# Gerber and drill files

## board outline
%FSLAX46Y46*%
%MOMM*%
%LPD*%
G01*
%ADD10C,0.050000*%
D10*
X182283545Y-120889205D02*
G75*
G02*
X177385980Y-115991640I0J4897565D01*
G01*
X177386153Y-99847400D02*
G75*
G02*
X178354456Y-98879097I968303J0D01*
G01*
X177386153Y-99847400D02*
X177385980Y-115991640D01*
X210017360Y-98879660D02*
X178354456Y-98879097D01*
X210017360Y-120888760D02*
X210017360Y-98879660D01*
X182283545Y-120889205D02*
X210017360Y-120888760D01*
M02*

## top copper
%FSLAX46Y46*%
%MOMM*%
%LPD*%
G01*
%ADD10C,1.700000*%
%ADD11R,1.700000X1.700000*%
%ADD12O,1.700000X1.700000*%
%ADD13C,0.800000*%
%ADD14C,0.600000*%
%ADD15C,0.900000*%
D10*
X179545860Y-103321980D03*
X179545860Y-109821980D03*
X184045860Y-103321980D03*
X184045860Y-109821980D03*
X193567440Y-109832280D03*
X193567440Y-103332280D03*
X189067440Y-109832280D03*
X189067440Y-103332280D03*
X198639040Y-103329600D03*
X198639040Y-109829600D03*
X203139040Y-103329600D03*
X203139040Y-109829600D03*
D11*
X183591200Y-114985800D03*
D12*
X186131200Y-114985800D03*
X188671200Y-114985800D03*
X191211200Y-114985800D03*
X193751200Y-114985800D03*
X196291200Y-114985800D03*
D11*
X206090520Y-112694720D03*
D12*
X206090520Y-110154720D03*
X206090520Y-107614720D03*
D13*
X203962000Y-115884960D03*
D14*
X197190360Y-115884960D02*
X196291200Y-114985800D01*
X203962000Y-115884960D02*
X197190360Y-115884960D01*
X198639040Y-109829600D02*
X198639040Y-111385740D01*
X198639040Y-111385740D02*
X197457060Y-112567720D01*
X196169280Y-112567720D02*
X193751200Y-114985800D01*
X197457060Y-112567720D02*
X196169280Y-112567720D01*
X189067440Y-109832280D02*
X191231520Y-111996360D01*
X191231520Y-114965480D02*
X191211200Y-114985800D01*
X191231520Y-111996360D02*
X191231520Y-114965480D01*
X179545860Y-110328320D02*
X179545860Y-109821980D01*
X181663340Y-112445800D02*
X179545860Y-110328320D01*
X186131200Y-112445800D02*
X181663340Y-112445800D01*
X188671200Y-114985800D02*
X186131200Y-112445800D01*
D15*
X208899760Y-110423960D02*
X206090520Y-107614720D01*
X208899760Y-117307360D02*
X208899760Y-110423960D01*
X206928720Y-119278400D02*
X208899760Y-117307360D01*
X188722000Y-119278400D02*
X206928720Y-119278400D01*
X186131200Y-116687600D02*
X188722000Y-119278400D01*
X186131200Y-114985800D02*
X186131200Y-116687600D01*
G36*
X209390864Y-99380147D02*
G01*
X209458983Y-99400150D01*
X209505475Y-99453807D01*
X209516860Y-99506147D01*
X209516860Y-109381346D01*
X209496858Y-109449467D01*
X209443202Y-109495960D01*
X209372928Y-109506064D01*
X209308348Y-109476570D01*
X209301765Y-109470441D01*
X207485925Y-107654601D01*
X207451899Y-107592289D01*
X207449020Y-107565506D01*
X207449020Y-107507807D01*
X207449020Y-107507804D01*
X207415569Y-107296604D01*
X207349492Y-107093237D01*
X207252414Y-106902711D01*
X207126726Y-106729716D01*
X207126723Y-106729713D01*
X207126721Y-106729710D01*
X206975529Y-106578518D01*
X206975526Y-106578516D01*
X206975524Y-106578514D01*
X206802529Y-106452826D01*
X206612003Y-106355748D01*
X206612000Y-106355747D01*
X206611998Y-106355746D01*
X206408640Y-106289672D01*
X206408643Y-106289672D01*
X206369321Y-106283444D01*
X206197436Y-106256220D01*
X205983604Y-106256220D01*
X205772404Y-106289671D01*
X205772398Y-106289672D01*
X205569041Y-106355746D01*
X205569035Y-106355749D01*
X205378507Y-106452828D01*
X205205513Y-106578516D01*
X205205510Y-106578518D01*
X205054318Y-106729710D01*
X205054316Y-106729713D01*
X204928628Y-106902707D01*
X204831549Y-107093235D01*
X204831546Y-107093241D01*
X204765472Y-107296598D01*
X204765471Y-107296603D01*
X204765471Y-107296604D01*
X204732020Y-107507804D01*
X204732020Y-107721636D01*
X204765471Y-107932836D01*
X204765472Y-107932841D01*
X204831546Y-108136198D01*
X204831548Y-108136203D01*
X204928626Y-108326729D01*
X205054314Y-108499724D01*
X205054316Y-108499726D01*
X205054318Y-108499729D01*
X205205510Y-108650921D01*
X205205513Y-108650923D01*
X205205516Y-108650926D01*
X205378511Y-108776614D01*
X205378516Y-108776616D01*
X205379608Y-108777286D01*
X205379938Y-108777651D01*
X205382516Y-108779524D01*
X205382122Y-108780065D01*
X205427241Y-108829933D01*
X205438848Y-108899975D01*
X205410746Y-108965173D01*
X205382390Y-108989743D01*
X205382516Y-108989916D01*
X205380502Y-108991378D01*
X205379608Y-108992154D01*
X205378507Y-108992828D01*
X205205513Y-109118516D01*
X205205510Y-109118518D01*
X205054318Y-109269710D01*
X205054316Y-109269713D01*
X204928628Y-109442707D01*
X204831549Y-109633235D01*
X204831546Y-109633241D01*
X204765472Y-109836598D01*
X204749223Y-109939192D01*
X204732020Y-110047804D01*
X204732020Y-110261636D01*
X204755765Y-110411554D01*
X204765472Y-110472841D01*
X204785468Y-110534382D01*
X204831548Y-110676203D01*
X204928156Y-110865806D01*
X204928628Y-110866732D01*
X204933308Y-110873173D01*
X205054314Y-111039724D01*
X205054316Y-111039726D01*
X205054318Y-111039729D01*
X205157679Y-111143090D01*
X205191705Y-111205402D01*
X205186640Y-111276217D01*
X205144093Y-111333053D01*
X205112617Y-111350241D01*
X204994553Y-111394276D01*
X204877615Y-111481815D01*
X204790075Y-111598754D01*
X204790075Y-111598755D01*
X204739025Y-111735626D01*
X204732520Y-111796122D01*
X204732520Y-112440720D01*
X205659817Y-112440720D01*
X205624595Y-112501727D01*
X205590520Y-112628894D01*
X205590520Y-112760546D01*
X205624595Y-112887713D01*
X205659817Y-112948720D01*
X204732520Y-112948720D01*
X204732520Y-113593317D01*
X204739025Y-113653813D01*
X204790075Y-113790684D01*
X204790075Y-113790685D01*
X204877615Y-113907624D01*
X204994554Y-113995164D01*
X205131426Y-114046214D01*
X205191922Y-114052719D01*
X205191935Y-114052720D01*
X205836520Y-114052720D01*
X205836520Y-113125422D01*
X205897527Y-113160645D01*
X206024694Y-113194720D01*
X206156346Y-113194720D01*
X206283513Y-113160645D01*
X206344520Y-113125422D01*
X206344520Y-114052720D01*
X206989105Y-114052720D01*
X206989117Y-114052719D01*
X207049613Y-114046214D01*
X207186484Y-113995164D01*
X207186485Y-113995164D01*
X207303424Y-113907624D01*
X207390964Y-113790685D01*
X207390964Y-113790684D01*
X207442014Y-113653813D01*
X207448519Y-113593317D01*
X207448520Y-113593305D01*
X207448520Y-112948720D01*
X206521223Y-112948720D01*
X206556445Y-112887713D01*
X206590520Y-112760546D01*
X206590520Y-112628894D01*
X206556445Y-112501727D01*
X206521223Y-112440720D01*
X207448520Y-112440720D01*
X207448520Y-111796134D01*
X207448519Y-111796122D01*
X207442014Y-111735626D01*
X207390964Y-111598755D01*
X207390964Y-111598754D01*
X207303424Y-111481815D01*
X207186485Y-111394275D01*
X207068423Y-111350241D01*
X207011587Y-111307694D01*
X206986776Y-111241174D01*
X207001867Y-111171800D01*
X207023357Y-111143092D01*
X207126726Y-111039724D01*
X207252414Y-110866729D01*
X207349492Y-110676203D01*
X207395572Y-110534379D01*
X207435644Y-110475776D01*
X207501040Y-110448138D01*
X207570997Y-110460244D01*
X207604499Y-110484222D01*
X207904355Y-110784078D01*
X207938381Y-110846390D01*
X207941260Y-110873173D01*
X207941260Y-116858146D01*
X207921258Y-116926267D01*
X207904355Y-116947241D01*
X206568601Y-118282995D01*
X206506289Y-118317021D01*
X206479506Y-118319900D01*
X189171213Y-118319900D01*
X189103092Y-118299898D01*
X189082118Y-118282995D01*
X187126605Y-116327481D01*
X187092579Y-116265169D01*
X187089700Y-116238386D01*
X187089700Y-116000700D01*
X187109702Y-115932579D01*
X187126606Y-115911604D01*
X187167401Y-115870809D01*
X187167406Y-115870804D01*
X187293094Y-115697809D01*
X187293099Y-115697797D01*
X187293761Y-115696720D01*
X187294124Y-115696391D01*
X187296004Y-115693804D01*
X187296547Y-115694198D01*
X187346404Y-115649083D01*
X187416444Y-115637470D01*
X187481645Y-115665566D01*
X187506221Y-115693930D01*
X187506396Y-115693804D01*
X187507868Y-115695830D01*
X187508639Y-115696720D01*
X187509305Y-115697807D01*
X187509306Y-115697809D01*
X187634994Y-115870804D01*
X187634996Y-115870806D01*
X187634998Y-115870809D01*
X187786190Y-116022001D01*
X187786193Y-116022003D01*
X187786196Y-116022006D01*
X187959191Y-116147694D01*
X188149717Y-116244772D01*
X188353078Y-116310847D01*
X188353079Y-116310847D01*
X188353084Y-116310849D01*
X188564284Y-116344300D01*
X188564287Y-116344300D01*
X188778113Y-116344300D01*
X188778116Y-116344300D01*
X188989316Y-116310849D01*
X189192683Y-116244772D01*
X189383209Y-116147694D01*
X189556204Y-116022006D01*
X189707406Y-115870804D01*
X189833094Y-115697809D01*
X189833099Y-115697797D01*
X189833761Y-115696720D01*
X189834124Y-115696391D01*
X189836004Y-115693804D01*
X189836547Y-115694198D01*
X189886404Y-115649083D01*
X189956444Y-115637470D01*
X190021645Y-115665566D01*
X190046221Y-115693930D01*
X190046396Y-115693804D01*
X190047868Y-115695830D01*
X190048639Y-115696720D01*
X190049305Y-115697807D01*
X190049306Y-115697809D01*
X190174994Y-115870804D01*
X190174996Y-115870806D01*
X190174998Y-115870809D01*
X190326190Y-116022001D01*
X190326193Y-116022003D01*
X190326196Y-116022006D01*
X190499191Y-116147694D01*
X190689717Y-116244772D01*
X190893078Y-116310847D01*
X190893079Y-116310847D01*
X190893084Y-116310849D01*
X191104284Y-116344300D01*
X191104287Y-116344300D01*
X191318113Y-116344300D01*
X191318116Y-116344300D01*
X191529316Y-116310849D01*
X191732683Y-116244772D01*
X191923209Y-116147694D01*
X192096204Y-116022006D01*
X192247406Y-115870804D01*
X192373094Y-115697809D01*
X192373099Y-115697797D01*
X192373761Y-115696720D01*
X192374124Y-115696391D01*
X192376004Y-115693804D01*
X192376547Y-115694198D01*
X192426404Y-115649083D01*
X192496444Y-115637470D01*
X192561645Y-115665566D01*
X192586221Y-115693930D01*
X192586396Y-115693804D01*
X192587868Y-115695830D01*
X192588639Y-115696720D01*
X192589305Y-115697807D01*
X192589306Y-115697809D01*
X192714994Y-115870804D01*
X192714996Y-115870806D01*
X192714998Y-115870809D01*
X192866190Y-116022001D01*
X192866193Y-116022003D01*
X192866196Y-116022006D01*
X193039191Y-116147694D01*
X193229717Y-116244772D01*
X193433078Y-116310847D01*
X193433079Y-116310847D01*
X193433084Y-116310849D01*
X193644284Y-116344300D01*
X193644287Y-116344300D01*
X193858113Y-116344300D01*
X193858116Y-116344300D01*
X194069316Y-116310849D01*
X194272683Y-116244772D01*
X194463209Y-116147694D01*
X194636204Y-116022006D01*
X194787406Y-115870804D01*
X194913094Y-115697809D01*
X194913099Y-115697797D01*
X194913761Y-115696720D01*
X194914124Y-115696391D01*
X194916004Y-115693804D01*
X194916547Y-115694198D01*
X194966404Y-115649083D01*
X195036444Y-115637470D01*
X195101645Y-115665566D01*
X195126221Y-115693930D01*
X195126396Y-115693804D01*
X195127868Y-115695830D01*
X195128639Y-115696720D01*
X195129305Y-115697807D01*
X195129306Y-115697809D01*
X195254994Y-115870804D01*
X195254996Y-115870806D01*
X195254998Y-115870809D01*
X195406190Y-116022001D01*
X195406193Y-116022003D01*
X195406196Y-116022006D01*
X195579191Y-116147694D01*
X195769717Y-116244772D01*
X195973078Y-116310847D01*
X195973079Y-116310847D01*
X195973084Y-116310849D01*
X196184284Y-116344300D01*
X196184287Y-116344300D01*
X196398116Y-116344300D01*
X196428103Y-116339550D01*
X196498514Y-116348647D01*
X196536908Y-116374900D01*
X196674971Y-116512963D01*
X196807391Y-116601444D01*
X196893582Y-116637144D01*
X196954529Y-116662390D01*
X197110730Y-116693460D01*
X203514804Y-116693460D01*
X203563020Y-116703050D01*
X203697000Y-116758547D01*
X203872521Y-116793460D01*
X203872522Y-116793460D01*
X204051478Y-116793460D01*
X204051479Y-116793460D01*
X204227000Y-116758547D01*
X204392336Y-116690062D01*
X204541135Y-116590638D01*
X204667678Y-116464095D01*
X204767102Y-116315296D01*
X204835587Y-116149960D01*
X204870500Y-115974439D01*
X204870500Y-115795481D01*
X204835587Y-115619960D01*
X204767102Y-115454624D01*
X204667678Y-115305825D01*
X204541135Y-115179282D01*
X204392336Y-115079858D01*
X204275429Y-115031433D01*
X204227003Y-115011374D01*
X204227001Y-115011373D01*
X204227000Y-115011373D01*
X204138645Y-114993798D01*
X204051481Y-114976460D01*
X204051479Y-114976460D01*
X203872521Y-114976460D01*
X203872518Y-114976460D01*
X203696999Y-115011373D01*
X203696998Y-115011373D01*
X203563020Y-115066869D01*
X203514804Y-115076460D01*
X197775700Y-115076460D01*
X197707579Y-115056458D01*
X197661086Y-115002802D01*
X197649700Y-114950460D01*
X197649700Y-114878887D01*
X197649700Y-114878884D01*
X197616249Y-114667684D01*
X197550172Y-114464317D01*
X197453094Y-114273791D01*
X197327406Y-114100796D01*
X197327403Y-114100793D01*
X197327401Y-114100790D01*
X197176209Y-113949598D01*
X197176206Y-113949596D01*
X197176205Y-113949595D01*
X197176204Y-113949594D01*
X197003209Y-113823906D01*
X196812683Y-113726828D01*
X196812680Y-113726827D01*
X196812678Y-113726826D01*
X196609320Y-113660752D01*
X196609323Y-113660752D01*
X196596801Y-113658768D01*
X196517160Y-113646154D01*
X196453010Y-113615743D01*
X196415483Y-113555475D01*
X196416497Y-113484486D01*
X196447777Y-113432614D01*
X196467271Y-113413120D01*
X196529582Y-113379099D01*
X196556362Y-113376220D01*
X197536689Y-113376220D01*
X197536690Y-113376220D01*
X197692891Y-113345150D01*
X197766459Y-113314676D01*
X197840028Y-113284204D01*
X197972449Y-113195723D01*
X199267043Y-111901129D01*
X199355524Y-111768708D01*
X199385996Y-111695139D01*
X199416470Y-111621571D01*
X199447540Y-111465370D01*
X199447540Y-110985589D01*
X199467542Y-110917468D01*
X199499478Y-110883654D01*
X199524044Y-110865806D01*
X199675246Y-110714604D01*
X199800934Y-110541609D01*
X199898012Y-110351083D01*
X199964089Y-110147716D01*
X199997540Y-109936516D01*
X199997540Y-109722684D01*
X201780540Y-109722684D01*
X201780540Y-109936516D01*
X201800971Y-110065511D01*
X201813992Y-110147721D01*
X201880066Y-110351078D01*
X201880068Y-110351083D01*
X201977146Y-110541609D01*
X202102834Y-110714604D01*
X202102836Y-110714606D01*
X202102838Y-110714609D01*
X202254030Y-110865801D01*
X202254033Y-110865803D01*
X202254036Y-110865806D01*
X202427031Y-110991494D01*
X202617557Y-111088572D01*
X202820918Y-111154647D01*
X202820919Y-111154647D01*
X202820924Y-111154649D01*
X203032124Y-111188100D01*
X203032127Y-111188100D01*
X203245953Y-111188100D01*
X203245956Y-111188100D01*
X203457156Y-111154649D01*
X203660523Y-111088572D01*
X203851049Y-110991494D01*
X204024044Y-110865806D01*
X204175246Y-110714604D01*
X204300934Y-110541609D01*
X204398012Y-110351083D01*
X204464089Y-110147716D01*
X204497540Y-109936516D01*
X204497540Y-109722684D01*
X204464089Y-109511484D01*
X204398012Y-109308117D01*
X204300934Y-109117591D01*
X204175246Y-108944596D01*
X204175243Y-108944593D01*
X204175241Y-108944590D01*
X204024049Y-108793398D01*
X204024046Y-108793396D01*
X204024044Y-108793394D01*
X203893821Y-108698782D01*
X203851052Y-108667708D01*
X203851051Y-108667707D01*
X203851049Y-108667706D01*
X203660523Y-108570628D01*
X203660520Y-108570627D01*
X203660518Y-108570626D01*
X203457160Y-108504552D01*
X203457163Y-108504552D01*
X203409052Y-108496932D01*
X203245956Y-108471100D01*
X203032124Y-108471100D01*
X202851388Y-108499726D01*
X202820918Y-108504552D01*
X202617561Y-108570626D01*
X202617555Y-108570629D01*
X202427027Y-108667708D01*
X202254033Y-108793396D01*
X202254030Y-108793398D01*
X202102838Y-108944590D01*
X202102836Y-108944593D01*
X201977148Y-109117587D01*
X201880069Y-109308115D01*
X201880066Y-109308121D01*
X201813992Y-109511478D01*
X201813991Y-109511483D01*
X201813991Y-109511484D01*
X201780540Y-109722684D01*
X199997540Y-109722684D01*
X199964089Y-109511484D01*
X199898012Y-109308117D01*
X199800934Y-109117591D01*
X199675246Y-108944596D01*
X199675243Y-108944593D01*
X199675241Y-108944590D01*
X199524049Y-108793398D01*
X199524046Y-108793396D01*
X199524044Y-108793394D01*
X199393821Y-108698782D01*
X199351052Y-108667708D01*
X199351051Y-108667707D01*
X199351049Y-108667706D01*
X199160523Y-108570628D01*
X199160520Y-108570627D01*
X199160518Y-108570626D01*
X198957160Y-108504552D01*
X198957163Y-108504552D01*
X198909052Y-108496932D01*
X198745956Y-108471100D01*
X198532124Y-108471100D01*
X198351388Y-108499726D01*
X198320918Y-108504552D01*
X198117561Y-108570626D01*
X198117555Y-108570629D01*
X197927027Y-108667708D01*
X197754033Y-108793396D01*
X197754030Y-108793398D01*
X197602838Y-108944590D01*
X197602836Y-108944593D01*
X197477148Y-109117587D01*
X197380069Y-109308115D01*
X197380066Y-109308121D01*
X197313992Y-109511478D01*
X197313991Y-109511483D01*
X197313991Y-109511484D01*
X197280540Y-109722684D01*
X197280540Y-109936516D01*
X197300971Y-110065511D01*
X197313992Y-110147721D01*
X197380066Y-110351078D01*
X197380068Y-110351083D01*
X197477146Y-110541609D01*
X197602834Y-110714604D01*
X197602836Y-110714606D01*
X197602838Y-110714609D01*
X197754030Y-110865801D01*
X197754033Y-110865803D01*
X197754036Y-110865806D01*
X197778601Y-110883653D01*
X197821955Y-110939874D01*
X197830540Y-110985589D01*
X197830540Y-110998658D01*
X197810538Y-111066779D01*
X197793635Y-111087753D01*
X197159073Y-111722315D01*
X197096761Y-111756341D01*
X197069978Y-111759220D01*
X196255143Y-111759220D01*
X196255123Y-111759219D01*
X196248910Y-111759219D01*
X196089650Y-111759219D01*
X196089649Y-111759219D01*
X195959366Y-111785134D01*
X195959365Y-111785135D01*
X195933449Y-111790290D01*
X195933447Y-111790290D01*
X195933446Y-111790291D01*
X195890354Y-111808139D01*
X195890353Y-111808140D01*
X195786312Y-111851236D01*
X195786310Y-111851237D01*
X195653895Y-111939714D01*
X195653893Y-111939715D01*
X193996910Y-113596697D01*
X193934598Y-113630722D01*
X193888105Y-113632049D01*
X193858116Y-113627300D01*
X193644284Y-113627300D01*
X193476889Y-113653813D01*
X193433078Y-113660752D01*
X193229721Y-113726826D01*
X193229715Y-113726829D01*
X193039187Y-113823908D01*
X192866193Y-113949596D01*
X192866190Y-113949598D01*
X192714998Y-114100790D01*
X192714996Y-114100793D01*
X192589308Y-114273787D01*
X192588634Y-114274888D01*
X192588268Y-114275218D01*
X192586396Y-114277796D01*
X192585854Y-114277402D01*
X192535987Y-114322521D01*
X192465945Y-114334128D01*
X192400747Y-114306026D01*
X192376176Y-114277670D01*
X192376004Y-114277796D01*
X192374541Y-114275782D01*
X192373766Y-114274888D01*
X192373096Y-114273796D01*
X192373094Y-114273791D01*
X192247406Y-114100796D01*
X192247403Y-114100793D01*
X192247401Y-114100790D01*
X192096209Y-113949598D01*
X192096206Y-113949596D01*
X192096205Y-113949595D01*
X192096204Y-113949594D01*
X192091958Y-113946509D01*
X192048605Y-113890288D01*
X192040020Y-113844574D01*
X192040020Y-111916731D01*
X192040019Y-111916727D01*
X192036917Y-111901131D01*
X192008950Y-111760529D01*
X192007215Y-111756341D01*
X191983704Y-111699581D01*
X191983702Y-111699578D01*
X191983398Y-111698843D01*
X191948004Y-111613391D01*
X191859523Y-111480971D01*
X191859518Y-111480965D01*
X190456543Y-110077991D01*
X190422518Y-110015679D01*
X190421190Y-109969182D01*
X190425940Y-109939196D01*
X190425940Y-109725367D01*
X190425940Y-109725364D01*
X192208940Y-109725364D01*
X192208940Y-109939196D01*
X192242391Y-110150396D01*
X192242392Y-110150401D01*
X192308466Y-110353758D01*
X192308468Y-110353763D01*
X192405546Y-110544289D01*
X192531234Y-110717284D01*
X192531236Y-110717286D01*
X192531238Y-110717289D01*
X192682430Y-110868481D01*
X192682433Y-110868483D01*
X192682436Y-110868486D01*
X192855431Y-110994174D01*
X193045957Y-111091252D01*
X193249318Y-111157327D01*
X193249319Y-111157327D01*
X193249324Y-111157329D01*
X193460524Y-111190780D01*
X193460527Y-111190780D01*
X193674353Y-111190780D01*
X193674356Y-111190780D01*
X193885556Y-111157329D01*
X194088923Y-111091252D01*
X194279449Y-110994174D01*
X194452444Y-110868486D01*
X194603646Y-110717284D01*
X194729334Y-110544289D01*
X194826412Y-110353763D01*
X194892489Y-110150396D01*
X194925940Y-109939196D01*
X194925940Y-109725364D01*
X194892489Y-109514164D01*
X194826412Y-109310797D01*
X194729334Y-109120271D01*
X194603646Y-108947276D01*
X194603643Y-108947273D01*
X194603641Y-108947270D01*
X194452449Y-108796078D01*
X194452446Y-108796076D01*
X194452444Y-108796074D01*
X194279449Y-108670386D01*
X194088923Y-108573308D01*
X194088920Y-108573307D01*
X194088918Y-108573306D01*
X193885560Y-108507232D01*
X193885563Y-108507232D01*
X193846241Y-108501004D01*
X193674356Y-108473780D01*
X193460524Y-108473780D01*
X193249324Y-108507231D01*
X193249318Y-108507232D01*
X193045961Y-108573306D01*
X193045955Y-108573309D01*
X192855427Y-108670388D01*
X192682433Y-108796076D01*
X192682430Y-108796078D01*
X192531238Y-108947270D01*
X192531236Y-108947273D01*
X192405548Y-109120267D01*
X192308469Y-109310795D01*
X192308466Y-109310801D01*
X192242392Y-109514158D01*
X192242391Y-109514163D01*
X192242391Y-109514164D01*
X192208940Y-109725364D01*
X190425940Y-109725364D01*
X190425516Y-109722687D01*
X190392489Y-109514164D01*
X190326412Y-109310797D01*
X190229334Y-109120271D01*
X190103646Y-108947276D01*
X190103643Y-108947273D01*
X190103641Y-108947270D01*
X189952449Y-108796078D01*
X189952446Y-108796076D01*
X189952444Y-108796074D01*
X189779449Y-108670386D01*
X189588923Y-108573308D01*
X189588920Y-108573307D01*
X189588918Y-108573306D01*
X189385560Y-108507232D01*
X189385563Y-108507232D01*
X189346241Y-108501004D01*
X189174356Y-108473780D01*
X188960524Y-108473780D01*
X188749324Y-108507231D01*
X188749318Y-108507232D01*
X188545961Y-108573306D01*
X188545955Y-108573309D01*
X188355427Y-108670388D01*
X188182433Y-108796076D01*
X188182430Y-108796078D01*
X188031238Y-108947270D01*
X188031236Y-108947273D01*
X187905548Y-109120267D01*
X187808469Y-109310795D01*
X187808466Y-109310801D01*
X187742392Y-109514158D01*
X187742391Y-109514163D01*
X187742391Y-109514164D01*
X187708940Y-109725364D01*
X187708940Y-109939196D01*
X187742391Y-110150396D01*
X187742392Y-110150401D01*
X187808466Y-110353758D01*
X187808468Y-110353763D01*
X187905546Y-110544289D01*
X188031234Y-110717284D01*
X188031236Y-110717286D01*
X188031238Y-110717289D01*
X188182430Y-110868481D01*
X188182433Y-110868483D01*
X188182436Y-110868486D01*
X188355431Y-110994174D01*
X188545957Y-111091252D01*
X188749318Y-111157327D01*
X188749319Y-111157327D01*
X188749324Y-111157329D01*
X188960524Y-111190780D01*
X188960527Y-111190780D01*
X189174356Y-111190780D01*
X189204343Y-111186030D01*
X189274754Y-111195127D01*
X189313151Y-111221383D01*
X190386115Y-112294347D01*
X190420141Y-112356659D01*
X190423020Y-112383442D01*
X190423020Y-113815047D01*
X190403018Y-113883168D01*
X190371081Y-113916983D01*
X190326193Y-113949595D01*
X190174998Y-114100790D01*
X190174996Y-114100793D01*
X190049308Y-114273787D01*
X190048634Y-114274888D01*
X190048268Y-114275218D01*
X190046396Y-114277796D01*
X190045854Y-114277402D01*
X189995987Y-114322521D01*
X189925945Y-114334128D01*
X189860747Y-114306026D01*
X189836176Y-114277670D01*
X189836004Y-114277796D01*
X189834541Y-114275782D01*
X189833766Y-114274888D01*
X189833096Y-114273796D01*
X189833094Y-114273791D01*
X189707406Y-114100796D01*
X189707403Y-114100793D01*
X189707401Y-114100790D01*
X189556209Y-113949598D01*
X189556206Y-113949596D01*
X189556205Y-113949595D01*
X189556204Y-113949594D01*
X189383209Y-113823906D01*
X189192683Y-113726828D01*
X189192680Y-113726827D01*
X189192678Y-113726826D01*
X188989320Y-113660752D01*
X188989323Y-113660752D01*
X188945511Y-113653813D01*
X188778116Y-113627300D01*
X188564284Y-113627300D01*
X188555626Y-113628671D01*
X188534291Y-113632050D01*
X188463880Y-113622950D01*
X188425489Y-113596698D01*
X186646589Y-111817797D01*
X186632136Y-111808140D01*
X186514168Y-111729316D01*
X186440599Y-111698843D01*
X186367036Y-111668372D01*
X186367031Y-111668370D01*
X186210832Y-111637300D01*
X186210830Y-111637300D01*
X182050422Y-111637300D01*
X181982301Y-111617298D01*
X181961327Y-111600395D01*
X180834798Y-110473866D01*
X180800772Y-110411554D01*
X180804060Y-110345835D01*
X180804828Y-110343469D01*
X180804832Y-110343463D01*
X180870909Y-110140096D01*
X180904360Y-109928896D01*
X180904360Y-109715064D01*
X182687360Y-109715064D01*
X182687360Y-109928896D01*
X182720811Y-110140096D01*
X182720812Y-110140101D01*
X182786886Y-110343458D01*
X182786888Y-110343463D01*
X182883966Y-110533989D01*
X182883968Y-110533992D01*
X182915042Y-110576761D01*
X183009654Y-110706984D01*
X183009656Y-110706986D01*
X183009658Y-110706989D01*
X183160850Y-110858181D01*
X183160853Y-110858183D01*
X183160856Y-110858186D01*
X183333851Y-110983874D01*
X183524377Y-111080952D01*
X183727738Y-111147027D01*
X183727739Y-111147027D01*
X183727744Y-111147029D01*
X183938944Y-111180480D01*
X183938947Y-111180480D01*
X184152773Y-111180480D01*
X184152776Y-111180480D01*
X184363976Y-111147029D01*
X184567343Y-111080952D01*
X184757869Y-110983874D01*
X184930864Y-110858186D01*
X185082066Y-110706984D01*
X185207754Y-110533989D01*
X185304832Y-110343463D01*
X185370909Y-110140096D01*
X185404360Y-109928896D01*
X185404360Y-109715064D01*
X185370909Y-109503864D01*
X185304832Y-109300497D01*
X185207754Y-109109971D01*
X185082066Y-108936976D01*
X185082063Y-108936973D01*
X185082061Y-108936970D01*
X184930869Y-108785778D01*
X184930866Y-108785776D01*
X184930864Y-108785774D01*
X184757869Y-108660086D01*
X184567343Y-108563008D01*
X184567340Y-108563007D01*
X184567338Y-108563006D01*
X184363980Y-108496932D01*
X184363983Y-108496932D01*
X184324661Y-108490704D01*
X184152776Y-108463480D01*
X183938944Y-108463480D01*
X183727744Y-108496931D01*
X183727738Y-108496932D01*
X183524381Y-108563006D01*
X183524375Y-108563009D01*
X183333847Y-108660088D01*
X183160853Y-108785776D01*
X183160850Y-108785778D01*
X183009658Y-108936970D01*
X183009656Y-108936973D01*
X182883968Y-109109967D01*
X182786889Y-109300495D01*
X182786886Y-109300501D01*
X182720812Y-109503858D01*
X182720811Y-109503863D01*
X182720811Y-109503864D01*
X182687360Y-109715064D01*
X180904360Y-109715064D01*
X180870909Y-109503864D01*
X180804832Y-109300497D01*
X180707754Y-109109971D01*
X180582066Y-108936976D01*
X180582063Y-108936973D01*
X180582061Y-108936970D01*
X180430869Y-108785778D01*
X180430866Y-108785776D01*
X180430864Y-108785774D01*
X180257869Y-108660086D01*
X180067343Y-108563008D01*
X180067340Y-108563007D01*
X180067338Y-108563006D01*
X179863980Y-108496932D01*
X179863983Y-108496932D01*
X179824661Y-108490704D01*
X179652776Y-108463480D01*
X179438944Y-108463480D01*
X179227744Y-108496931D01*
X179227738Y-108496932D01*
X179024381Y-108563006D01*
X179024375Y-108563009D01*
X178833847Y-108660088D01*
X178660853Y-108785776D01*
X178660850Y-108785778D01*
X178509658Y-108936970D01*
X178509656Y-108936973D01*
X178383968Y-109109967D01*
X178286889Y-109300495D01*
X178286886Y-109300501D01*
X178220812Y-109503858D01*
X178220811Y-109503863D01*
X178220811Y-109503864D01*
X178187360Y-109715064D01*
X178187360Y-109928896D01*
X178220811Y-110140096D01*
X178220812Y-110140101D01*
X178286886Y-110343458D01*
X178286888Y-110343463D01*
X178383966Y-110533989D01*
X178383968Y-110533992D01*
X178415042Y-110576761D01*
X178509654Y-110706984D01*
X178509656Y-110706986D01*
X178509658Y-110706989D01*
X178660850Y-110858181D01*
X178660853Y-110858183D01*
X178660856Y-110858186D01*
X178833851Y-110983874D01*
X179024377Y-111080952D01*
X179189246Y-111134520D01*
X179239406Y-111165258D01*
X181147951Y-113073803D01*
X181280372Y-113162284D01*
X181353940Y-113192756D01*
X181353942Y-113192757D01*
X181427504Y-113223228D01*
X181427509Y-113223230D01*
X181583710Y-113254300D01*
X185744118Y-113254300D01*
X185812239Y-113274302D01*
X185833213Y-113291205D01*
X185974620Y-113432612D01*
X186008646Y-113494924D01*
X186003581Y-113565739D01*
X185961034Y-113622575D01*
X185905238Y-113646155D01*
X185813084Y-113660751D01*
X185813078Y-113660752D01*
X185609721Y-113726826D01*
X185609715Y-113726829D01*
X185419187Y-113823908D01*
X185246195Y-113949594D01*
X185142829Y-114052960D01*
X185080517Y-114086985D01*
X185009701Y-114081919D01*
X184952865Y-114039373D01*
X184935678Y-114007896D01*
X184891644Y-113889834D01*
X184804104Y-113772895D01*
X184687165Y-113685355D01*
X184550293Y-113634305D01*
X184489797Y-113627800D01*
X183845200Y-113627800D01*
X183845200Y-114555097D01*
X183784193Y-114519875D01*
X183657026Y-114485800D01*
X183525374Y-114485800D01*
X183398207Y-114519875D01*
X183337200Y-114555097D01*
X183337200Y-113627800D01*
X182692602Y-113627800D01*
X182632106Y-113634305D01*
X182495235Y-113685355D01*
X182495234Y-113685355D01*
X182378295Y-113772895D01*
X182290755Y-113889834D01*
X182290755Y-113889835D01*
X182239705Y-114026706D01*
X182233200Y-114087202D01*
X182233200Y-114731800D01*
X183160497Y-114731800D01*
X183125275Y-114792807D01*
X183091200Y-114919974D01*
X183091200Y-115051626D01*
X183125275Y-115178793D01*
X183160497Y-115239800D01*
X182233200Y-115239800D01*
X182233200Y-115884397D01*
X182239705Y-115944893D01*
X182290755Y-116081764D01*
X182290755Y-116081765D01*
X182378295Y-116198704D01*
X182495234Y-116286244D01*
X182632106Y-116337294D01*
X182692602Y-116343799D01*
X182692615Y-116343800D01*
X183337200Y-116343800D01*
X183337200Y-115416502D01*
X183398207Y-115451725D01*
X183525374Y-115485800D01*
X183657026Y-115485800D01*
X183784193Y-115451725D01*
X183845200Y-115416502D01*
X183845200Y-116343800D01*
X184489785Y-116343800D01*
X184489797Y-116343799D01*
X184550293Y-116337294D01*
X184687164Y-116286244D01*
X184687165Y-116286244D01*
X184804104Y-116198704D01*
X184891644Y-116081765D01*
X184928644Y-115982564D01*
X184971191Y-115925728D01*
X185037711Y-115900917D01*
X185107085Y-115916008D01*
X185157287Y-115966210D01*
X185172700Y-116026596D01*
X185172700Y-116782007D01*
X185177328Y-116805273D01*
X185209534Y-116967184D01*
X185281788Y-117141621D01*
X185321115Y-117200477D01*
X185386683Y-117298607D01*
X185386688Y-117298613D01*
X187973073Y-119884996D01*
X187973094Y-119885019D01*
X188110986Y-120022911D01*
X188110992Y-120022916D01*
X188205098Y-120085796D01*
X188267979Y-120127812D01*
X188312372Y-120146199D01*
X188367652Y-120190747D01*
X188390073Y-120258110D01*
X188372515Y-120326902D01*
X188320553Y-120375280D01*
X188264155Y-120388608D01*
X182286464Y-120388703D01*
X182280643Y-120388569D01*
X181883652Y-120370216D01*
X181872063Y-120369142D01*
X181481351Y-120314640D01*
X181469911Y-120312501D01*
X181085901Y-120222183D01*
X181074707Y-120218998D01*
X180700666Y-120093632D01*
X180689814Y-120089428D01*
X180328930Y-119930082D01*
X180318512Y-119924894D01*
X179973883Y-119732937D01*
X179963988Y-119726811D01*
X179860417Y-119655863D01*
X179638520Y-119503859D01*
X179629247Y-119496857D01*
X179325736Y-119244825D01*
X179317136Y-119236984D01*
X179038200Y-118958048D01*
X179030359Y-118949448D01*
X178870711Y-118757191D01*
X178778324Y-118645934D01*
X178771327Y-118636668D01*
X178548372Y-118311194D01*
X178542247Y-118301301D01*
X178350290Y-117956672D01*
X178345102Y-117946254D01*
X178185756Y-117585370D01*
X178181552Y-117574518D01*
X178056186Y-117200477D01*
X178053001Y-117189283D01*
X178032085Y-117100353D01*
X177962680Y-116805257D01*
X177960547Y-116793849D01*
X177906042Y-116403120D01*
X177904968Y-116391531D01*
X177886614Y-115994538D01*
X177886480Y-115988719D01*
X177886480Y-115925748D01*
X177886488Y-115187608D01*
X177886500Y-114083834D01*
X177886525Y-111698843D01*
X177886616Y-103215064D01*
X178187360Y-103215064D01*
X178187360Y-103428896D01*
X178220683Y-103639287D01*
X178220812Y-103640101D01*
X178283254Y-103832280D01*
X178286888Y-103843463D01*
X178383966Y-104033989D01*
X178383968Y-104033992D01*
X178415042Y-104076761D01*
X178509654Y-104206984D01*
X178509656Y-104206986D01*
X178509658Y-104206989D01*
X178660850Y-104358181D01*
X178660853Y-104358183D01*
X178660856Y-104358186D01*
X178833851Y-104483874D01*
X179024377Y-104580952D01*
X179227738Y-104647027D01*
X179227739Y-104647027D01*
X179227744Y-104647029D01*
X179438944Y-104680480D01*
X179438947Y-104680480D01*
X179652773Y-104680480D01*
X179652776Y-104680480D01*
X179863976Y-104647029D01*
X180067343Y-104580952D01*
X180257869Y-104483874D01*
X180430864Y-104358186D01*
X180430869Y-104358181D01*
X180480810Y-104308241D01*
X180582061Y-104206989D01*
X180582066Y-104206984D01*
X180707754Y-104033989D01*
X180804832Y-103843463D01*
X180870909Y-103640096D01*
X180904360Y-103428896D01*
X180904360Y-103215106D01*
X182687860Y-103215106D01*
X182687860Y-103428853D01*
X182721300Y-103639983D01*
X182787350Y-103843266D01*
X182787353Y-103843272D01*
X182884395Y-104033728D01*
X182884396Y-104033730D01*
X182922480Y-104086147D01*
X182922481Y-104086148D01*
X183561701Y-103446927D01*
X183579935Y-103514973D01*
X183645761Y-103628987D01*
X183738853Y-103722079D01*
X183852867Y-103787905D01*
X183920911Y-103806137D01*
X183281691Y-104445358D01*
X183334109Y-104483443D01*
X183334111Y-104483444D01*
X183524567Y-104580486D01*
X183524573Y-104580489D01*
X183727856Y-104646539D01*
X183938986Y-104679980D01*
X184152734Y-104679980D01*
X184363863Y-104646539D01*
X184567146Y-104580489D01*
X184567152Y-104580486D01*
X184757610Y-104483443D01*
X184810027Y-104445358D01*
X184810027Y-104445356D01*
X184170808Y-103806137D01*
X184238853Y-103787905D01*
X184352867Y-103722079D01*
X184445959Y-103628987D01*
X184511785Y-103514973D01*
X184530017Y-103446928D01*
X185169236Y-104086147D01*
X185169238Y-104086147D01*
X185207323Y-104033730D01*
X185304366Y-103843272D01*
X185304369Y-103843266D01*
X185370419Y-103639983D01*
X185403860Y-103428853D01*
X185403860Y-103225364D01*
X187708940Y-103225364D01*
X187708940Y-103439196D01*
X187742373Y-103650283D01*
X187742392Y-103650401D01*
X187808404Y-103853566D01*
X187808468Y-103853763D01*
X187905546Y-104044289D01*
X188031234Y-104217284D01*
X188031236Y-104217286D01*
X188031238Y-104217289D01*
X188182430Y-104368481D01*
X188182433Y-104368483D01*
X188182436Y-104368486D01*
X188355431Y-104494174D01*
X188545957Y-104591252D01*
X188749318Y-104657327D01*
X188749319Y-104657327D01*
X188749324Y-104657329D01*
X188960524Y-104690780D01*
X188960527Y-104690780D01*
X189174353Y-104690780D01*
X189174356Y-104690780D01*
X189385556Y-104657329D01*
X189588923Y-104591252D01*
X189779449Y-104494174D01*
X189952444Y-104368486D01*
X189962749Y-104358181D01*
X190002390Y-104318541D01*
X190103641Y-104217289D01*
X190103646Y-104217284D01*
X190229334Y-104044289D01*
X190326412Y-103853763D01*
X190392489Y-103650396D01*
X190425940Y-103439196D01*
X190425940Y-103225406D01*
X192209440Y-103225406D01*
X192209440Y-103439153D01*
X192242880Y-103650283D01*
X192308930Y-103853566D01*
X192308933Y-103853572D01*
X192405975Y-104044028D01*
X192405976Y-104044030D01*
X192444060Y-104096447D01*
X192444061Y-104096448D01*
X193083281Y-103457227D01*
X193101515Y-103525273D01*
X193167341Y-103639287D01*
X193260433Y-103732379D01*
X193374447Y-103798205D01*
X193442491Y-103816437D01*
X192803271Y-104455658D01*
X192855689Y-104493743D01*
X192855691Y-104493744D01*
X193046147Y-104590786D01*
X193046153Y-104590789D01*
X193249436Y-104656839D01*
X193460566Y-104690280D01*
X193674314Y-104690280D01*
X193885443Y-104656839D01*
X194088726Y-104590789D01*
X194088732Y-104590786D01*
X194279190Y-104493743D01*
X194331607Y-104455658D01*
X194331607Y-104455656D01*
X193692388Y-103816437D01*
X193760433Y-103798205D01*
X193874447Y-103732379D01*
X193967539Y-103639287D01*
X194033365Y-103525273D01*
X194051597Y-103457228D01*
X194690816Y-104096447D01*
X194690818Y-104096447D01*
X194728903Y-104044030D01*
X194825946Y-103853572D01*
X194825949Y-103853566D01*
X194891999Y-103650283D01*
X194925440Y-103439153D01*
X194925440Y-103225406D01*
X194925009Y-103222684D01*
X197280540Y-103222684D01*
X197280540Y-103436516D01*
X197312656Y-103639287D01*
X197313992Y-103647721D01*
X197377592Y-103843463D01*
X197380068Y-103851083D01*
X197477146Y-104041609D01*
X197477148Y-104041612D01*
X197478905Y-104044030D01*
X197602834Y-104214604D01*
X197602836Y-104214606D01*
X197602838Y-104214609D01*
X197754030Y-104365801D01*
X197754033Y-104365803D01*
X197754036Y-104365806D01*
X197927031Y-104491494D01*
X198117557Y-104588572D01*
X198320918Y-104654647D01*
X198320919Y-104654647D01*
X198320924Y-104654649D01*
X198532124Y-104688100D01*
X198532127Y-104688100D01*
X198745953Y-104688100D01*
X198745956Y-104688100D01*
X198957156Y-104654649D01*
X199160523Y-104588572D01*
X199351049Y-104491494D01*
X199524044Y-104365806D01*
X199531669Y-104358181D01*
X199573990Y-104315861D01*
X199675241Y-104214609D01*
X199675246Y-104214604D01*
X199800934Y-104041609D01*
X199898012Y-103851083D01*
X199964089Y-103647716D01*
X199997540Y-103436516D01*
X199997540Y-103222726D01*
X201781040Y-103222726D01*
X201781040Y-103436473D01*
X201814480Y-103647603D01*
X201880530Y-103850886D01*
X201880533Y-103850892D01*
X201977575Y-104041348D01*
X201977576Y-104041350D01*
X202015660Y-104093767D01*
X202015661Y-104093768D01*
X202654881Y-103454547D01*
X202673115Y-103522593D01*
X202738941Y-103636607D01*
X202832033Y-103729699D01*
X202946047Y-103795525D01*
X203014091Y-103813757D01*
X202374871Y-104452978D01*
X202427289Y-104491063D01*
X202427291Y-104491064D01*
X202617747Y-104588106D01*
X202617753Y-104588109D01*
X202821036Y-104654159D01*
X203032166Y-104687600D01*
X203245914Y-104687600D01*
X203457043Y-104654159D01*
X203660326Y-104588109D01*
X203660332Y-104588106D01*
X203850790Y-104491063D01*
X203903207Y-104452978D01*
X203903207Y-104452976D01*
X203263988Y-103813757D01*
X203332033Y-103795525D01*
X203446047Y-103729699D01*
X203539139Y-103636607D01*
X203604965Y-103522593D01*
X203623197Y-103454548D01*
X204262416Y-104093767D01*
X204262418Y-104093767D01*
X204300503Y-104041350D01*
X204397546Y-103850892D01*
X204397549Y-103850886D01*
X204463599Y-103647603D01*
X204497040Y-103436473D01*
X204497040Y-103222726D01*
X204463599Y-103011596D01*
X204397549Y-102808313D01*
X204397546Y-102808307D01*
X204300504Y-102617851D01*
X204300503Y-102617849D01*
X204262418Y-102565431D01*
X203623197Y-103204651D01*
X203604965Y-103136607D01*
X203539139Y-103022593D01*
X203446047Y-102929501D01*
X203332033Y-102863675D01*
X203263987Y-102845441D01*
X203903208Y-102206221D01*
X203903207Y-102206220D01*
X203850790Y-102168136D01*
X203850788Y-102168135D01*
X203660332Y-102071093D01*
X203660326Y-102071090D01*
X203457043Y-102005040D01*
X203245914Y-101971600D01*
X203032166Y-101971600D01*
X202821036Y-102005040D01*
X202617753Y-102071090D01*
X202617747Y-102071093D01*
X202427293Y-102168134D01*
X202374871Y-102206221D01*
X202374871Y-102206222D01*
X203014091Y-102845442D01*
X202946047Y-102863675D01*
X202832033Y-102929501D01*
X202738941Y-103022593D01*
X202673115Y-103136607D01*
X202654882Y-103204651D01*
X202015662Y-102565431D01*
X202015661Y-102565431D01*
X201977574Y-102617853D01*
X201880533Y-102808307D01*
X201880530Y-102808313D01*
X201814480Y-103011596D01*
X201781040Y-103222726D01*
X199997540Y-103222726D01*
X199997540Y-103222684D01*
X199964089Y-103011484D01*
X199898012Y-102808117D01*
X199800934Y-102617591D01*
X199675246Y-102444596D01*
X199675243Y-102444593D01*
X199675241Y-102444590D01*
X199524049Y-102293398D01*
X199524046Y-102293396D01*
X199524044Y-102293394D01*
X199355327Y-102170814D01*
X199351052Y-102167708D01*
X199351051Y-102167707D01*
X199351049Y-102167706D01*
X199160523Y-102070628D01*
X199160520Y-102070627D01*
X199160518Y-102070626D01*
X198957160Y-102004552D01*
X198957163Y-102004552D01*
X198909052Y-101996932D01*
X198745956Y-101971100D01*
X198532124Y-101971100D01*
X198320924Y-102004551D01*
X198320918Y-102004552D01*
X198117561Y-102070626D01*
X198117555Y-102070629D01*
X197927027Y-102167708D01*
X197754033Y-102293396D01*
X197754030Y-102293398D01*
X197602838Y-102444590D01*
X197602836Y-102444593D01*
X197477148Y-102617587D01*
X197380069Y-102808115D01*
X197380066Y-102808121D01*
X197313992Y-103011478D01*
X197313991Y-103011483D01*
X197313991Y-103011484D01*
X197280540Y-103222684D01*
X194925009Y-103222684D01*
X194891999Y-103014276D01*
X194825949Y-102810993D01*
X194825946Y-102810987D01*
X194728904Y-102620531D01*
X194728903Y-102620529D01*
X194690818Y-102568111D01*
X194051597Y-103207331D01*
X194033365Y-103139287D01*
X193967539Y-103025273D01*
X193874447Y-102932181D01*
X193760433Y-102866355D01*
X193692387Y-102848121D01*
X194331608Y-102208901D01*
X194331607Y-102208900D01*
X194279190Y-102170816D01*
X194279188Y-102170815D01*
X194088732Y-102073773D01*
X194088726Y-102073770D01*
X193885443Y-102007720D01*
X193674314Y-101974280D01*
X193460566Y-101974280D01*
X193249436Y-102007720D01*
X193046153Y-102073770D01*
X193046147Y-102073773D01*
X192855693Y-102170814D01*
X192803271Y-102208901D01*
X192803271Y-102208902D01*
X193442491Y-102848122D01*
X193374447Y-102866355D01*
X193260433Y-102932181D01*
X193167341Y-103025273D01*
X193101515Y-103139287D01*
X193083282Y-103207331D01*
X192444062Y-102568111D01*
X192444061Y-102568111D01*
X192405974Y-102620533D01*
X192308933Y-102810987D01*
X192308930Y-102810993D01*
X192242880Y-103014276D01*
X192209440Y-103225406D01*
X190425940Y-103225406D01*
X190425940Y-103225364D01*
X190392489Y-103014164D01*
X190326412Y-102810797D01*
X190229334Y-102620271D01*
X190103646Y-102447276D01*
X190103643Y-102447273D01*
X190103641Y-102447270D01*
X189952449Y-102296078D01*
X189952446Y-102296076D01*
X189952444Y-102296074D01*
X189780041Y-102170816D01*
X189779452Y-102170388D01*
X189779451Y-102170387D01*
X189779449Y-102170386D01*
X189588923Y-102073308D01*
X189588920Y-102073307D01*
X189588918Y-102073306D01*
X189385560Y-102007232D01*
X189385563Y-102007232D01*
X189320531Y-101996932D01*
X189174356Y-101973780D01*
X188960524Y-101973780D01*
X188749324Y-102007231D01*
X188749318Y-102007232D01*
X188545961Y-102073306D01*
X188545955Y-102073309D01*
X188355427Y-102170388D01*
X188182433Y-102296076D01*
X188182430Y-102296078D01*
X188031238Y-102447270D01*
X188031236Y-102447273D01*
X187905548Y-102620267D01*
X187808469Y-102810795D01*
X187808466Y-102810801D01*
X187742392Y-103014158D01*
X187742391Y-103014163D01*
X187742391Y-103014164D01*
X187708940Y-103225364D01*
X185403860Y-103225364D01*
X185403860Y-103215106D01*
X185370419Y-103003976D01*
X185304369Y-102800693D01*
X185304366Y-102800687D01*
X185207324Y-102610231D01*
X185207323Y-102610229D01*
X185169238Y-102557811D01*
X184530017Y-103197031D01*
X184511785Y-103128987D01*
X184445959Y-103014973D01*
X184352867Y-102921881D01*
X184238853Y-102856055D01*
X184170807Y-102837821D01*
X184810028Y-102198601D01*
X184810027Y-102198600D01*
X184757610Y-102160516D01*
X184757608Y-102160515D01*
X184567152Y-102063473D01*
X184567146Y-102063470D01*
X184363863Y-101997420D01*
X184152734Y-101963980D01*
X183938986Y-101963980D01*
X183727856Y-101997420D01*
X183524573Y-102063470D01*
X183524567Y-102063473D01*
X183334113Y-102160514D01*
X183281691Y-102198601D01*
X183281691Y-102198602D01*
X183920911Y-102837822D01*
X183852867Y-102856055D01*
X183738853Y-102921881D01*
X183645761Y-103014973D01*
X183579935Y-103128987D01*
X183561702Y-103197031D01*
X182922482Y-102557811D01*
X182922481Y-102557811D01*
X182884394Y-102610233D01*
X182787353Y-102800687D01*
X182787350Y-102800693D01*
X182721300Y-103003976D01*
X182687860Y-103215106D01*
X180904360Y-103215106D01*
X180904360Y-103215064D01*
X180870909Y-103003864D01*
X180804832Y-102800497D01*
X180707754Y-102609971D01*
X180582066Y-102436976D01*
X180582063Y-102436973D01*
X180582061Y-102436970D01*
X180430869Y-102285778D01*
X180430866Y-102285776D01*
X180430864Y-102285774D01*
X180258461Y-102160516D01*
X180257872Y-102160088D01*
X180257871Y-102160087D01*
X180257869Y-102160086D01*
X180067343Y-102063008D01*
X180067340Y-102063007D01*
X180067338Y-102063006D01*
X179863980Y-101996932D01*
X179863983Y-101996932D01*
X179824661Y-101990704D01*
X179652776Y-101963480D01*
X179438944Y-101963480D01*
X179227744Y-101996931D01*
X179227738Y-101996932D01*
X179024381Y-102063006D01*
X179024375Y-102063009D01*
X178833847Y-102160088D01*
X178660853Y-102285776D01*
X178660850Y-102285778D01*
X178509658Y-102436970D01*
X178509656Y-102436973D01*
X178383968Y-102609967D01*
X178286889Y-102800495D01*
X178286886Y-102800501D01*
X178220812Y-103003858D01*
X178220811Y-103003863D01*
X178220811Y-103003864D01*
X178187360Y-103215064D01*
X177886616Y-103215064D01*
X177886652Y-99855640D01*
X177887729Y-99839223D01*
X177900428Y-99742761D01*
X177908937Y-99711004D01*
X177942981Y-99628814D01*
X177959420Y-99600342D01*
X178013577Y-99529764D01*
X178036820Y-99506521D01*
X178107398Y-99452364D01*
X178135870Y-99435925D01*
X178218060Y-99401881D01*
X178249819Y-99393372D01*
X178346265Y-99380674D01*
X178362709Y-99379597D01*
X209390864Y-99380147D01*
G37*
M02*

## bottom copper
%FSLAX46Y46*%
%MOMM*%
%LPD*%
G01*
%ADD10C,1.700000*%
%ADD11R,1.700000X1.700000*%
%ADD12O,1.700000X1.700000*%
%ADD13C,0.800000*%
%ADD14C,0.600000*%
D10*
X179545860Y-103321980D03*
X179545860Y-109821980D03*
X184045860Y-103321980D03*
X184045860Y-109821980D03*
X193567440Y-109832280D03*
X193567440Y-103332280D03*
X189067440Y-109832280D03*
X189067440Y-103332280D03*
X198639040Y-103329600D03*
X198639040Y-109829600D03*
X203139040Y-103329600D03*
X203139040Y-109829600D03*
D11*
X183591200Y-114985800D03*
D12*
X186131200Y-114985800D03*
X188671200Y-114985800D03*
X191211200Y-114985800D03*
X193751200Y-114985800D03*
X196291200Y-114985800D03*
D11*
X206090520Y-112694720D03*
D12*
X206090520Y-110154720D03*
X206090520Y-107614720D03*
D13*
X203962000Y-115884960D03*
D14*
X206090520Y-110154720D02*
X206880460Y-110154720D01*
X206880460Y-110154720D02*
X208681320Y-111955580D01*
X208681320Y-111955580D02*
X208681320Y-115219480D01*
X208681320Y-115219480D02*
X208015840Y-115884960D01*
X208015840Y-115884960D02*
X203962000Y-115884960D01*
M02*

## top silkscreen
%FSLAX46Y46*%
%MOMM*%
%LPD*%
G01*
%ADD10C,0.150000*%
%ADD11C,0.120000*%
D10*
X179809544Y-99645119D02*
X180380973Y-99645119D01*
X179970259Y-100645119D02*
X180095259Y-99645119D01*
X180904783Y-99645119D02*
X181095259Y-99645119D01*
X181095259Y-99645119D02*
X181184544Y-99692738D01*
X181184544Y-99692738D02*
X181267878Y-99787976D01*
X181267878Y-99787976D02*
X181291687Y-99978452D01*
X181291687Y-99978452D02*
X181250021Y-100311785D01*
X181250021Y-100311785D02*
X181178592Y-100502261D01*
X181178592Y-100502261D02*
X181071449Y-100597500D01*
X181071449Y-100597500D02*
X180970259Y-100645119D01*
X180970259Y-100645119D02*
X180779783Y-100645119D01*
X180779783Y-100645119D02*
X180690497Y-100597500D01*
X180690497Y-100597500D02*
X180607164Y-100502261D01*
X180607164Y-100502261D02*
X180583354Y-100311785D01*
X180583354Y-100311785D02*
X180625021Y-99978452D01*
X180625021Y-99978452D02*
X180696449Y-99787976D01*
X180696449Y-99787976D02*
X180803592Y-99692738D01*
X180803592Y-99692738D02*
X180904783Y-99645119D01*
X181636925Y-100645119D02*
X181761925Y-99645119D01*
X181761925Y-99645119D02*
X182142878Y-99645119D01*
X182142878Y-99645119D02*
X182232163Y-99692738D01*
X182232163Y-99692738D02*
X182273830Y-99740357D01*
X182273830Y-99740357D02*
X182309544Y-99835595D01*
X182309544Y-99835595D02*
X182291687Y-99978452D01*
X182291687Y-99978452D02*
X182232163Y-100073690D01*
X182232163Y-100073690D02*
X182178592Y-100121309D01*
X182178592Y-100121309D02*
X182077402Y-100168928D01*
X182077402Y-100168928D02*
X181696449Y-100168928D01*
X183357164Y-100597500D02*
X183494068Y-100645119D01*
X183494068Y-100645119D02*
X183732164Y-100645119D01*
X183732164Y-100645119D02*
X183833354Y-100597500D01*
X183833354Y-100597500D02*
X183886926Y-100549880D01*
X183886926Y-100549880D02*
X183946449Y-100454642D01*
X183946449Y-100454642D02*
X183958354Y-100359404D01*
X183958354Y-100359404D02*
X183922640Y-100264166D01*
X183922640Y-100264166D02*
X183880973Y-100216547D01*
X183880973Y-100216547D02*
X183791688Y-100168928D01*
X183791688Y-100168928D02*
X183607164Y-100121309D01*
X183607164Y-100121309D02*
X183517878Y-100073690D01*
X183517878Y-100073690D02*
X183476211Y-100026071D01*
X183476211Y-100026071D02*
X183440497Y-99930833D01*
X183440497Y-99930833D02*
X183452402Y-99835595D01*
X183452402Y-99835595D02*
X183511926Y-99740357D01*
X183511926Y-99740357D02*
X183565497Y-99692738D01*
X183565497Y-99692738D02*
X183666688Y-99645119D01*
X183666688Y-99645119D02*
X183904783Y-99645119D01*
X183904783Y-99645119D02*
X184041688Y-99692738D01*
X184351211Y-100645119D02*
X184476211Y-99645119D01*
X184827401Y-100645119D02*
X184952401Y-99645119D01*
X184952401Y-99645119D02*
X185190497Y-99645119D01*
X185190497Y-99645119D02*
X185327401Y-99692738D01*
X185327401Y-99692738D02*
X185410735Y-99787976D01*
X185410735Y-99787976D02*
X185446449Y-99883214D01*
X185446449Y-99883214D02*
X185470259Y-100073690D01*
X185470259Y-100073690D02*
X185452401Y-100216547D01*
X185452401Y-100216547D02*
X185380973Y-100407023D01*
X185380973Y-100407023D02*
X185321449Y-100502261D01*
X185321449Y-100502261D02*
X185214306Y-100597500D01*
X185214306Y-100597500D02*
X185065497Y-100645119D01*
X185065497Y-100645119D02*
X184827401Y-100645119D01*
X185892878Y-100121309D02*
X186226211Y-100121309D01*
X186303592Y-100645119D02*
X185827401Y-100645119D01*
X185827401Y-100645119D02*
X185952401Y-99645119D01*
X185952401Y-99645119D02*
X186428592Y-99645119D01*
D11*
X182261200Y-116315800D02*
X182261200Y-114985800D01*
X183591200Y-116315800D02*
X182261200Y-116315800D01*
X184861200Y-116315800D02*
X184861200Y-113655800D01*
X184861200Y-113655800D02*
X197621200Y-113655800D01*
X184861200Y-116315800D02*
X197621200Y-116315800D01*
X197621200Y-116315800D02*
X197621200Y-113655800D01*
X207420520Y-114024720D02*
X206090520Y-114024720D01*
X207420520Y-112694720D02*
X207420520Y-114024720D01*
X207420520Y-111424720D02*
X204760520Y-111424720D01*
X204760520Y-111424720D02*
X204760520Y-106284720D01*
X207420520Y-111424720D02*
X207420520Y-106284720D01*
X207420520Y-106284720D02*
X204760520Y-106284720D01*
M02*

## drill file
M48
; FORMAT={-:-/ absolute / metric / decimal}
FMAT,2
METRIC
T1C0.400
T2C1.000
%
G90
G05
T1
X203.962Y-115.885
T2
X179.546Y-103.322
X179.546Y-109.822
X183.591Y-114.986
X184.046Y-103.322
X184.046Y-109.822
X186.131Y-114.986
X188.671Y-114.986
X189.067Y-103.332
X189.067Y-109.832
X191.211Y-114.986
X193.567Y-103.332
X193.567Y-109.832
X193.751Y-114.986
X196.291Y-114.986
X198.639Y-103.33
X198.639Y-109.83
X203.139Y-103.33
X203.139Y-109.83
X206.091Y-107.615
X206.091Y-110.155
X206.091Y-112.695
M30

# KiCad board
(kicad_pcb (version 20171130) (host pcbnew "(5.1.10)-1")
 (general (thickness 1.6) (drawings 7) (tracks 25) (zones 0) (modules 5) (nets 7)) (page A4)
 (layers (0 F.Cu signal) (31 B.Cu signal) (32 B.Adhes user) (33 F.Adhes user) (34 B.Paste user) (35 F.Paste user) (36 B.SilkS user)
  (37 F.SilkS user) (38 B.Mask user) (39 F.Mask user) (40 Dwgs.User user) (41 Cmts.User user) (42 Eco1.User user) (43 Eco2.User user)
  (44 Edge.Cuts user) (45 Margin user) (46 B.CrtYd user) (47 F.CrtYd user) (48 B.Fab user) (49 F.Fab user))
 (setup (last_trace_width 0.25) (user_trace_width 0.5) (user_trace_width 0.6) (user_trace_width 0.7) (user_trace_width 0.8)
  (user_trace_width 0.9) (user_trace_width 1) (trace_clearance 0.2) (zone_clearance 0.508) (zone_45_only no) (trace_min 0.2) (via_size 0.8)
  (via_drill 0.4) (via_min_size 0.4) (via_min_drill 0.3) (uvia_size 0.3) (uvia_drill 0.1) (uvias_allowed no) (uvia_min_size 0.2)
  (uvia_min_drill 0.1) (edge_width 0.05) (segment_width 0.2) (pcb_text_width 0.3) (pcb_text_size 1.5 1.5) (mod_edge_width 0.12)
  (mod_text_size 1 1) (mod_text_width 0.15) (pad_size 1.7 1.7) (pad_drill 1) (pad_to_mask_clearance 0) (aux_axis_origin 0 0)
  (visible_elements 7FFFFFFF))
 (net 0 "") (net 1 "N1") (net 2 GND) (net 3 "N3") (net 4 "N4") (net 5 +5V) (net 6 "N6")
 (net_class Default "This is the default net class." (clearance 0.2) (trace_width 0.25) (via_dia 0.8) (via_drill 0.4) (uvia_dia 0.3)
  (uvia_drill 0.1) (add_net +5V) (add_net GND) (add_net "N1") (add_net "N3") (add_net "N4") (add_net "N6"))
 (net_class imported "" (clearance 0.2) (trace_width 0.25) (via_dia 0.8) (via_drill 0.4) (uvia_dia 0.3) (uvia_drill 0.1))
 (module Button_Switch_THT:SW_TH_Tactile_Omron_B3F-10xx (layer B.Cu) (at 184.04586 109.82198 90)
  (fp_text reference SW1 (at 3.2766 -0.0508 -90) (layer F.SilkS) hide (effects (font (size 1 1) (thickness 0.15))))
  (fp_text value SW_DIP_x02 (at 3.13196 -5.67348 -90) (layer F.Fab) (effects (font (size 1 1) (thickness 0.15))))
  (pad 4 thru_hole circle (at 6.5 -4.5 90) (size 1.7 1.7) (drill 1) (layers *.Cu *.Mask))
  (pad 3 thru_hole circle (at 0 -4.5 90) (size 1.7 1.7) (drill 1) (layers *.Cu *.Mask) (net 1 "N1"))
  (pad 2 thru_hole circle (at 6.5 0 90) (size 1.7 1.7) (drill 1) (layers *.Cu *.Mask) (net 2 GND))
  (pad 1 thru_hole circle (at 0 0 90) (size 1.7 1.7) (drill 1) (layers *.Cu *.Mask)))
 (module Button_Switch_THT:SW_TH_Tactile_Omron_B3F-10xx (layer B.Cu) (at 193.56744 109.83228 90)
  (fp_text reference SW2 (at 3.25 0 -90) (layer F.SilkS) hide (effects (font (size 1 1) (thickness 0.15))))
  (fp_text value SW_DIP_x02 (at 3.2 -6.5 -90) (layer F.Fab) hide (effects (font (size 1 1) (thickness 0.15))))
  (pad 1 thru_hole circle (at 0 0 90) (size 1.7 1.7) (drill 1) (layers *.Cu *.Mask))
  (pad 2 thru_hole circle (at 6.5 0 90) (size 1.7 1.7) (drill 1) (layers *.Cu *.Mask) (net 2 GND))
  (pad 3 thru_hole circle (at 0 -4.5 90) (size 1.7 1.7) (drill 1) (layers *.Cu *.Mask) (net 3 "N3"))
  (pad 4 thru_hole circle (at 6.5 -4.5 90) (size 1.7 1.7) (drill 1) (layers *.Cu *.Mask)))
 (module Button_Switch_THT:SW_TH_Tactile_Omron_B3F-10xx (layer B.Cu) (at 203.13904 109.8296 90)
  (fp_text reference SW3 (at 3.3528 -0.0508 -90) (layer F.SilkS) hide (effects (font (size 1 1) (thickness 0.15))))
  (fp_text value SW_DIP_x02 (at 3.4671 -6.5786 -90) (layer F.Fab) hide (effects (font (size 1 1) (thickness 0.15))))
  (pad 4 thru_hole circle (at 6.5 -4.5 90) (size 1.7 1.7) (drill 1) (layers *.Cu *.Mask))
  (pad 3 thru_hole circle (at 0 -4.5 90) (size 1.7 1.7) (drill 1) (layers *.Cu *.Mask) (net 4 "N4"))
  (pad 2 thru_hole circle (at 6.5 0 90) (size 1.7 1.7) (drill 1) (layers *.Cu *.Mask) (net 2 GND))
  (pad 1 thru_hole circle (at 0 0 90) (size 1.7 1.7) (drill 1) (layers *.Cu *.Mask)))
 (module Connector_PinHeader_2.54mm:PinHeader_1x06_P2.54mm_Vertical (layer F.Cu) (at 183.5912 114.9858 90)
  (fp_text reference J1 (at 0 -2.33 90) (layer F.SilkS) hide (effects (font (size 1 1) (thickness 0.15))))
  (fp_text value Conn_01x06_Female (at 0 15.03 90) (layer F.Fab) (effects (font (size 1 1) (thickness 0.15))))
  (fp_line (start -1.33 -1.33) (end 0 -1.33) (layer F.SilkS) (width 0.12))
  (fp_line (start -1.33 0) (end -1.33 -1.33) (layer F.SilkS) (width 0.12))
  (fp_line (start -1.33 1.27) (end 1.33 1.27) (layer F.SilkS) (width 0.12))
  (fp_line (start 1.33 1.27) (end 1.33 14.03) (layer F.SilkS) (width 0.12))
  (fp_line (start -1.33 1.27) (end -1.33 14.03) (layer F.SilkS) (width 0.12))
  (fp_line (start -1.33 14.03) (end 1.33 14.03) (layer F.SilkS) (width 0.12))
  (pad 1 thru_hole rect (at 0 0 90) (size 1.7 1.7) (drill 1) (layers *.Cu *.Mask) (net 2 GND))
  (pad 2 thru_hole oval (at 0 2.54 90) (size 1.7 1.7) (drill 1) (layers *.Cu *.Mask) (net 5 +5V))
  (pad 3 thru_hole oval (at 0 5.08 90) (size 1.7 1.7) (drill 1) (layers *.Cu *.Mask) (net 1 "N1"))
  (pad 4 thru_hole oval (at 0 7.62 90) (size 1.7 1.7) (drill 1) (layers *.Cu *.Mask) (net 3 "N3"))
  (pad 5 thru_hole oval (at 0 10.16 90) (size 1.7 1.7) (drill 1) (layers *.Cu *.Mask) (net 4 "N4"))
  (pad 6 thru_hole oval (at 0 12.7 90) (size 1.7 1.7) (drill 1) (layers *.Cu *.Mask) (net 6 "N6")))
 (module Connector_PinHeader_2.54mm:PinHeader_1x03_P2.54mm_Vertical (layer F.Cu) (at 206.09052 112.69472 180)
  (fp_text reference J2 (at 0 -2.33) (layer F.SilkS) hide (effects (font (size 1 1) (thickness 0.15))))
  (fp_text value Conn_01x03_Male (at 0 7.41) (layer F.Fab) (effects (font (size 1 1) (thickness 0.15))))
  (fp_line (start -1.33 -1.33) (end 0 -1.33) (layer F.SilkS) (width 0.12))
  (fp_line (start -1.33 0) (end -1.33 -1.33) (layer F.SilkS) (width 0.12))
  (fp_line (start -1.33 1.27) (end 1.33 1.27) (layer F.SilkS) (width 0.12))
  (fp_line (start 1.33 1.27) (end 1.33 6.41) (layer F.SilkS) (width 0.12))
  (fp_line (start -1.33 1.27) (end -1.33 6.41) (layer F.SilkS) (width 0.12))
  (fp_line (start -1.33 6.41) (end 1.33 6.41) (layer F.SilkS) (width 0.12))
  (pad 1 thru_hole rect (at 0 0 180) (size 1.7 1.7) (drill 1) (layers *.Cu *.Mask) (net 2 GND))
  (pad 2 thru_hole oval (at 0 2.54 180) (size 1.7 1.7) (drill 1) (layers *.Cu *.Mask) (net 6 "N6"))
  (pad 3 thru_hole oval (at 0 5.08 180) (size 1.7 1.7) (drill 1) (layers *.Cu *.Mask) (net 5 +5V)))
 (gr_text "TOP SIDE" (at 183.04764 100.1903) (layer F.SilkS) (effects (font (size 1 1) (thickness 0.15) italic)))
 (gr_arc (start 182.283545 115.99164) (end 177.38598 115.99164) (angle -90) (layer Edge.Cuts) (width 0.05))
 (gr_arc (start 178.354456 99.8474) (end 178.354456 98.879097) (angle -90) (layer Edge.Cuts) (width 0.05))
 (gr_line (start 177.386153 99.8474) (end 177.38598 115.99164) (layer Edge.Cuts) (width 0.05))
 (gr_line (start 210.01736 98.87966) (end 178.354456 98.879097) (layer Edge.Cuts) (width 0.05))
 (gr_line (start 210.01736 120.88876) (end 210.01736 98.87966) (layer Edge.Cuts) (width 0.05))
 (gr_line (start 182.283545 120.889205) (end 210.01736 120.88876) (layer Edge.Cuts) (width 0.05))
 (segment (start 206.09052 110.15472) (end 206.88046 110.15472) (width 0.6) (layer B.Cu) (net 6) (status 30))
 (segment (start 206.88046 110.15472) (end 208.68132 111.95558) (width 0.6) (layer B.Cu) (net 6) (status 10))
 (segment (start 208.68132 111.95558) (end 208.68132 115.21948) (width 0.6) (layer B.Cu) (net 6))
 (segment (start 208.68132 115.21948) (end 208.01584 115.88496) (width 0.6) (layer B.Cu) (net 6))
 (segment (start 208.01584 115.88496) (end 203.962 115.88496) (width 0.6) (layer B.Cu) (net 6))
 (via (at 203.962 115.88496) (size 0.8) (drill 0.4) (layers F.Cu B.Cu) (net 6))
 (segment (start 197.19036 115.88496) (end 196.2912 114.9858) (width 0.6) (layer F.Cu) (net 6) (status 20))
 (segment (start 203.962 115.88496) (end 197.19036 115.88496) (width 0.6) (layer F.Cu) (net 6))
 (segment (start 198.63904 109.8296) (end 198.63904 111.38574) (width 0.6) (layer F.Cu) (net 4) (status 10))
 (segment (start 198.63904 111.38574) (end 197.45706 112.56772) (width 0.6) (layer F.Cu) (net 4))
 (segment (start 196.16928 112.56772) (end 193.7512 114.9858) (width 0.6) (layer F.Cu) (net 4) (status 20))
 (segment (start 197.45706 112.56772) (end 196.16928 112.56772) (width 0.6) (layer F.Cu) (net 4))
 (segment (start 189.06744 109.83228) (end 191.23152 111.99636) (width 0.6) (layer F.Cu) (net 3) (status 10))
 (segment (start 191.23152 114.96548) (end 191.2112 114.9858) (width 0.6) (layer F.Cu) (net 3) (status 30))
 (segment (start 191.23152 111.99636) (end 191.23152 114.96548) (width 0.6) (layer F.Cu) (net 3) (status 20))
 (segment (start 179.54586 110.32832) (end 179.54586 109.82198) (width 0.6) (layer F.Cu) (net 1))
 (segment (start 181.66334 112.4458) (end 179.54586 110.32832) (width 0.6) (layer F.Cu) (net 1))
 (segment (start 186.1312 112.4458) (end 181.66334 112.4458) (width 0.6) (layer F.Cu) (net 1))
 (segment (start 188.6712 114.9858) (end 186.1312 112.4458) (width 0.6) (layer F.Cu) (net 1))
 (segment (start 208.89976 110.42396) (end 206.09052 107.61472) (width 0.9) (layer F.Cu) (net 5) (status 20))
 (segment (start 208.89976 117.30736) (end 208.89976 110.42396) (width 0.9) (layer F.Cu) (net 5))
 (segment (start 206.92872 119.2784) (end 208.89976 117.30736) (width 0.9) (layer F.Cu) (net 5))
 (segment (start 188.722 119.2784) (end 206.92872 119.2784) (width 0.9) (layer F.Cu) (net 5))
 (segment (start 186.1312 116.6876) (end 188.722 119.2784) (width 0.9) (layer F.Cu) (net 5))
 (segment (start 186.1312 114.9858) (end 186.1312 116.6876) (width 0.9) (layer F.Cu) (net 5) (status 10))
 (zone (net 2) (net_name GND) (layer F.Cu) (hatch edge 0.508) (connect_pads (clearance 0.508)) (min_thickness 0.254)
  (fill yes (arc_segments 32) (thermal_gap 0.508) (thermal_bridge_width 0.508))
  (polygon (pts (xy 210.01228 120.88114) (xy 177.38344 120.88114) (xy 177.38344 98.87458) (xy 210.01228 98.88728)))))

